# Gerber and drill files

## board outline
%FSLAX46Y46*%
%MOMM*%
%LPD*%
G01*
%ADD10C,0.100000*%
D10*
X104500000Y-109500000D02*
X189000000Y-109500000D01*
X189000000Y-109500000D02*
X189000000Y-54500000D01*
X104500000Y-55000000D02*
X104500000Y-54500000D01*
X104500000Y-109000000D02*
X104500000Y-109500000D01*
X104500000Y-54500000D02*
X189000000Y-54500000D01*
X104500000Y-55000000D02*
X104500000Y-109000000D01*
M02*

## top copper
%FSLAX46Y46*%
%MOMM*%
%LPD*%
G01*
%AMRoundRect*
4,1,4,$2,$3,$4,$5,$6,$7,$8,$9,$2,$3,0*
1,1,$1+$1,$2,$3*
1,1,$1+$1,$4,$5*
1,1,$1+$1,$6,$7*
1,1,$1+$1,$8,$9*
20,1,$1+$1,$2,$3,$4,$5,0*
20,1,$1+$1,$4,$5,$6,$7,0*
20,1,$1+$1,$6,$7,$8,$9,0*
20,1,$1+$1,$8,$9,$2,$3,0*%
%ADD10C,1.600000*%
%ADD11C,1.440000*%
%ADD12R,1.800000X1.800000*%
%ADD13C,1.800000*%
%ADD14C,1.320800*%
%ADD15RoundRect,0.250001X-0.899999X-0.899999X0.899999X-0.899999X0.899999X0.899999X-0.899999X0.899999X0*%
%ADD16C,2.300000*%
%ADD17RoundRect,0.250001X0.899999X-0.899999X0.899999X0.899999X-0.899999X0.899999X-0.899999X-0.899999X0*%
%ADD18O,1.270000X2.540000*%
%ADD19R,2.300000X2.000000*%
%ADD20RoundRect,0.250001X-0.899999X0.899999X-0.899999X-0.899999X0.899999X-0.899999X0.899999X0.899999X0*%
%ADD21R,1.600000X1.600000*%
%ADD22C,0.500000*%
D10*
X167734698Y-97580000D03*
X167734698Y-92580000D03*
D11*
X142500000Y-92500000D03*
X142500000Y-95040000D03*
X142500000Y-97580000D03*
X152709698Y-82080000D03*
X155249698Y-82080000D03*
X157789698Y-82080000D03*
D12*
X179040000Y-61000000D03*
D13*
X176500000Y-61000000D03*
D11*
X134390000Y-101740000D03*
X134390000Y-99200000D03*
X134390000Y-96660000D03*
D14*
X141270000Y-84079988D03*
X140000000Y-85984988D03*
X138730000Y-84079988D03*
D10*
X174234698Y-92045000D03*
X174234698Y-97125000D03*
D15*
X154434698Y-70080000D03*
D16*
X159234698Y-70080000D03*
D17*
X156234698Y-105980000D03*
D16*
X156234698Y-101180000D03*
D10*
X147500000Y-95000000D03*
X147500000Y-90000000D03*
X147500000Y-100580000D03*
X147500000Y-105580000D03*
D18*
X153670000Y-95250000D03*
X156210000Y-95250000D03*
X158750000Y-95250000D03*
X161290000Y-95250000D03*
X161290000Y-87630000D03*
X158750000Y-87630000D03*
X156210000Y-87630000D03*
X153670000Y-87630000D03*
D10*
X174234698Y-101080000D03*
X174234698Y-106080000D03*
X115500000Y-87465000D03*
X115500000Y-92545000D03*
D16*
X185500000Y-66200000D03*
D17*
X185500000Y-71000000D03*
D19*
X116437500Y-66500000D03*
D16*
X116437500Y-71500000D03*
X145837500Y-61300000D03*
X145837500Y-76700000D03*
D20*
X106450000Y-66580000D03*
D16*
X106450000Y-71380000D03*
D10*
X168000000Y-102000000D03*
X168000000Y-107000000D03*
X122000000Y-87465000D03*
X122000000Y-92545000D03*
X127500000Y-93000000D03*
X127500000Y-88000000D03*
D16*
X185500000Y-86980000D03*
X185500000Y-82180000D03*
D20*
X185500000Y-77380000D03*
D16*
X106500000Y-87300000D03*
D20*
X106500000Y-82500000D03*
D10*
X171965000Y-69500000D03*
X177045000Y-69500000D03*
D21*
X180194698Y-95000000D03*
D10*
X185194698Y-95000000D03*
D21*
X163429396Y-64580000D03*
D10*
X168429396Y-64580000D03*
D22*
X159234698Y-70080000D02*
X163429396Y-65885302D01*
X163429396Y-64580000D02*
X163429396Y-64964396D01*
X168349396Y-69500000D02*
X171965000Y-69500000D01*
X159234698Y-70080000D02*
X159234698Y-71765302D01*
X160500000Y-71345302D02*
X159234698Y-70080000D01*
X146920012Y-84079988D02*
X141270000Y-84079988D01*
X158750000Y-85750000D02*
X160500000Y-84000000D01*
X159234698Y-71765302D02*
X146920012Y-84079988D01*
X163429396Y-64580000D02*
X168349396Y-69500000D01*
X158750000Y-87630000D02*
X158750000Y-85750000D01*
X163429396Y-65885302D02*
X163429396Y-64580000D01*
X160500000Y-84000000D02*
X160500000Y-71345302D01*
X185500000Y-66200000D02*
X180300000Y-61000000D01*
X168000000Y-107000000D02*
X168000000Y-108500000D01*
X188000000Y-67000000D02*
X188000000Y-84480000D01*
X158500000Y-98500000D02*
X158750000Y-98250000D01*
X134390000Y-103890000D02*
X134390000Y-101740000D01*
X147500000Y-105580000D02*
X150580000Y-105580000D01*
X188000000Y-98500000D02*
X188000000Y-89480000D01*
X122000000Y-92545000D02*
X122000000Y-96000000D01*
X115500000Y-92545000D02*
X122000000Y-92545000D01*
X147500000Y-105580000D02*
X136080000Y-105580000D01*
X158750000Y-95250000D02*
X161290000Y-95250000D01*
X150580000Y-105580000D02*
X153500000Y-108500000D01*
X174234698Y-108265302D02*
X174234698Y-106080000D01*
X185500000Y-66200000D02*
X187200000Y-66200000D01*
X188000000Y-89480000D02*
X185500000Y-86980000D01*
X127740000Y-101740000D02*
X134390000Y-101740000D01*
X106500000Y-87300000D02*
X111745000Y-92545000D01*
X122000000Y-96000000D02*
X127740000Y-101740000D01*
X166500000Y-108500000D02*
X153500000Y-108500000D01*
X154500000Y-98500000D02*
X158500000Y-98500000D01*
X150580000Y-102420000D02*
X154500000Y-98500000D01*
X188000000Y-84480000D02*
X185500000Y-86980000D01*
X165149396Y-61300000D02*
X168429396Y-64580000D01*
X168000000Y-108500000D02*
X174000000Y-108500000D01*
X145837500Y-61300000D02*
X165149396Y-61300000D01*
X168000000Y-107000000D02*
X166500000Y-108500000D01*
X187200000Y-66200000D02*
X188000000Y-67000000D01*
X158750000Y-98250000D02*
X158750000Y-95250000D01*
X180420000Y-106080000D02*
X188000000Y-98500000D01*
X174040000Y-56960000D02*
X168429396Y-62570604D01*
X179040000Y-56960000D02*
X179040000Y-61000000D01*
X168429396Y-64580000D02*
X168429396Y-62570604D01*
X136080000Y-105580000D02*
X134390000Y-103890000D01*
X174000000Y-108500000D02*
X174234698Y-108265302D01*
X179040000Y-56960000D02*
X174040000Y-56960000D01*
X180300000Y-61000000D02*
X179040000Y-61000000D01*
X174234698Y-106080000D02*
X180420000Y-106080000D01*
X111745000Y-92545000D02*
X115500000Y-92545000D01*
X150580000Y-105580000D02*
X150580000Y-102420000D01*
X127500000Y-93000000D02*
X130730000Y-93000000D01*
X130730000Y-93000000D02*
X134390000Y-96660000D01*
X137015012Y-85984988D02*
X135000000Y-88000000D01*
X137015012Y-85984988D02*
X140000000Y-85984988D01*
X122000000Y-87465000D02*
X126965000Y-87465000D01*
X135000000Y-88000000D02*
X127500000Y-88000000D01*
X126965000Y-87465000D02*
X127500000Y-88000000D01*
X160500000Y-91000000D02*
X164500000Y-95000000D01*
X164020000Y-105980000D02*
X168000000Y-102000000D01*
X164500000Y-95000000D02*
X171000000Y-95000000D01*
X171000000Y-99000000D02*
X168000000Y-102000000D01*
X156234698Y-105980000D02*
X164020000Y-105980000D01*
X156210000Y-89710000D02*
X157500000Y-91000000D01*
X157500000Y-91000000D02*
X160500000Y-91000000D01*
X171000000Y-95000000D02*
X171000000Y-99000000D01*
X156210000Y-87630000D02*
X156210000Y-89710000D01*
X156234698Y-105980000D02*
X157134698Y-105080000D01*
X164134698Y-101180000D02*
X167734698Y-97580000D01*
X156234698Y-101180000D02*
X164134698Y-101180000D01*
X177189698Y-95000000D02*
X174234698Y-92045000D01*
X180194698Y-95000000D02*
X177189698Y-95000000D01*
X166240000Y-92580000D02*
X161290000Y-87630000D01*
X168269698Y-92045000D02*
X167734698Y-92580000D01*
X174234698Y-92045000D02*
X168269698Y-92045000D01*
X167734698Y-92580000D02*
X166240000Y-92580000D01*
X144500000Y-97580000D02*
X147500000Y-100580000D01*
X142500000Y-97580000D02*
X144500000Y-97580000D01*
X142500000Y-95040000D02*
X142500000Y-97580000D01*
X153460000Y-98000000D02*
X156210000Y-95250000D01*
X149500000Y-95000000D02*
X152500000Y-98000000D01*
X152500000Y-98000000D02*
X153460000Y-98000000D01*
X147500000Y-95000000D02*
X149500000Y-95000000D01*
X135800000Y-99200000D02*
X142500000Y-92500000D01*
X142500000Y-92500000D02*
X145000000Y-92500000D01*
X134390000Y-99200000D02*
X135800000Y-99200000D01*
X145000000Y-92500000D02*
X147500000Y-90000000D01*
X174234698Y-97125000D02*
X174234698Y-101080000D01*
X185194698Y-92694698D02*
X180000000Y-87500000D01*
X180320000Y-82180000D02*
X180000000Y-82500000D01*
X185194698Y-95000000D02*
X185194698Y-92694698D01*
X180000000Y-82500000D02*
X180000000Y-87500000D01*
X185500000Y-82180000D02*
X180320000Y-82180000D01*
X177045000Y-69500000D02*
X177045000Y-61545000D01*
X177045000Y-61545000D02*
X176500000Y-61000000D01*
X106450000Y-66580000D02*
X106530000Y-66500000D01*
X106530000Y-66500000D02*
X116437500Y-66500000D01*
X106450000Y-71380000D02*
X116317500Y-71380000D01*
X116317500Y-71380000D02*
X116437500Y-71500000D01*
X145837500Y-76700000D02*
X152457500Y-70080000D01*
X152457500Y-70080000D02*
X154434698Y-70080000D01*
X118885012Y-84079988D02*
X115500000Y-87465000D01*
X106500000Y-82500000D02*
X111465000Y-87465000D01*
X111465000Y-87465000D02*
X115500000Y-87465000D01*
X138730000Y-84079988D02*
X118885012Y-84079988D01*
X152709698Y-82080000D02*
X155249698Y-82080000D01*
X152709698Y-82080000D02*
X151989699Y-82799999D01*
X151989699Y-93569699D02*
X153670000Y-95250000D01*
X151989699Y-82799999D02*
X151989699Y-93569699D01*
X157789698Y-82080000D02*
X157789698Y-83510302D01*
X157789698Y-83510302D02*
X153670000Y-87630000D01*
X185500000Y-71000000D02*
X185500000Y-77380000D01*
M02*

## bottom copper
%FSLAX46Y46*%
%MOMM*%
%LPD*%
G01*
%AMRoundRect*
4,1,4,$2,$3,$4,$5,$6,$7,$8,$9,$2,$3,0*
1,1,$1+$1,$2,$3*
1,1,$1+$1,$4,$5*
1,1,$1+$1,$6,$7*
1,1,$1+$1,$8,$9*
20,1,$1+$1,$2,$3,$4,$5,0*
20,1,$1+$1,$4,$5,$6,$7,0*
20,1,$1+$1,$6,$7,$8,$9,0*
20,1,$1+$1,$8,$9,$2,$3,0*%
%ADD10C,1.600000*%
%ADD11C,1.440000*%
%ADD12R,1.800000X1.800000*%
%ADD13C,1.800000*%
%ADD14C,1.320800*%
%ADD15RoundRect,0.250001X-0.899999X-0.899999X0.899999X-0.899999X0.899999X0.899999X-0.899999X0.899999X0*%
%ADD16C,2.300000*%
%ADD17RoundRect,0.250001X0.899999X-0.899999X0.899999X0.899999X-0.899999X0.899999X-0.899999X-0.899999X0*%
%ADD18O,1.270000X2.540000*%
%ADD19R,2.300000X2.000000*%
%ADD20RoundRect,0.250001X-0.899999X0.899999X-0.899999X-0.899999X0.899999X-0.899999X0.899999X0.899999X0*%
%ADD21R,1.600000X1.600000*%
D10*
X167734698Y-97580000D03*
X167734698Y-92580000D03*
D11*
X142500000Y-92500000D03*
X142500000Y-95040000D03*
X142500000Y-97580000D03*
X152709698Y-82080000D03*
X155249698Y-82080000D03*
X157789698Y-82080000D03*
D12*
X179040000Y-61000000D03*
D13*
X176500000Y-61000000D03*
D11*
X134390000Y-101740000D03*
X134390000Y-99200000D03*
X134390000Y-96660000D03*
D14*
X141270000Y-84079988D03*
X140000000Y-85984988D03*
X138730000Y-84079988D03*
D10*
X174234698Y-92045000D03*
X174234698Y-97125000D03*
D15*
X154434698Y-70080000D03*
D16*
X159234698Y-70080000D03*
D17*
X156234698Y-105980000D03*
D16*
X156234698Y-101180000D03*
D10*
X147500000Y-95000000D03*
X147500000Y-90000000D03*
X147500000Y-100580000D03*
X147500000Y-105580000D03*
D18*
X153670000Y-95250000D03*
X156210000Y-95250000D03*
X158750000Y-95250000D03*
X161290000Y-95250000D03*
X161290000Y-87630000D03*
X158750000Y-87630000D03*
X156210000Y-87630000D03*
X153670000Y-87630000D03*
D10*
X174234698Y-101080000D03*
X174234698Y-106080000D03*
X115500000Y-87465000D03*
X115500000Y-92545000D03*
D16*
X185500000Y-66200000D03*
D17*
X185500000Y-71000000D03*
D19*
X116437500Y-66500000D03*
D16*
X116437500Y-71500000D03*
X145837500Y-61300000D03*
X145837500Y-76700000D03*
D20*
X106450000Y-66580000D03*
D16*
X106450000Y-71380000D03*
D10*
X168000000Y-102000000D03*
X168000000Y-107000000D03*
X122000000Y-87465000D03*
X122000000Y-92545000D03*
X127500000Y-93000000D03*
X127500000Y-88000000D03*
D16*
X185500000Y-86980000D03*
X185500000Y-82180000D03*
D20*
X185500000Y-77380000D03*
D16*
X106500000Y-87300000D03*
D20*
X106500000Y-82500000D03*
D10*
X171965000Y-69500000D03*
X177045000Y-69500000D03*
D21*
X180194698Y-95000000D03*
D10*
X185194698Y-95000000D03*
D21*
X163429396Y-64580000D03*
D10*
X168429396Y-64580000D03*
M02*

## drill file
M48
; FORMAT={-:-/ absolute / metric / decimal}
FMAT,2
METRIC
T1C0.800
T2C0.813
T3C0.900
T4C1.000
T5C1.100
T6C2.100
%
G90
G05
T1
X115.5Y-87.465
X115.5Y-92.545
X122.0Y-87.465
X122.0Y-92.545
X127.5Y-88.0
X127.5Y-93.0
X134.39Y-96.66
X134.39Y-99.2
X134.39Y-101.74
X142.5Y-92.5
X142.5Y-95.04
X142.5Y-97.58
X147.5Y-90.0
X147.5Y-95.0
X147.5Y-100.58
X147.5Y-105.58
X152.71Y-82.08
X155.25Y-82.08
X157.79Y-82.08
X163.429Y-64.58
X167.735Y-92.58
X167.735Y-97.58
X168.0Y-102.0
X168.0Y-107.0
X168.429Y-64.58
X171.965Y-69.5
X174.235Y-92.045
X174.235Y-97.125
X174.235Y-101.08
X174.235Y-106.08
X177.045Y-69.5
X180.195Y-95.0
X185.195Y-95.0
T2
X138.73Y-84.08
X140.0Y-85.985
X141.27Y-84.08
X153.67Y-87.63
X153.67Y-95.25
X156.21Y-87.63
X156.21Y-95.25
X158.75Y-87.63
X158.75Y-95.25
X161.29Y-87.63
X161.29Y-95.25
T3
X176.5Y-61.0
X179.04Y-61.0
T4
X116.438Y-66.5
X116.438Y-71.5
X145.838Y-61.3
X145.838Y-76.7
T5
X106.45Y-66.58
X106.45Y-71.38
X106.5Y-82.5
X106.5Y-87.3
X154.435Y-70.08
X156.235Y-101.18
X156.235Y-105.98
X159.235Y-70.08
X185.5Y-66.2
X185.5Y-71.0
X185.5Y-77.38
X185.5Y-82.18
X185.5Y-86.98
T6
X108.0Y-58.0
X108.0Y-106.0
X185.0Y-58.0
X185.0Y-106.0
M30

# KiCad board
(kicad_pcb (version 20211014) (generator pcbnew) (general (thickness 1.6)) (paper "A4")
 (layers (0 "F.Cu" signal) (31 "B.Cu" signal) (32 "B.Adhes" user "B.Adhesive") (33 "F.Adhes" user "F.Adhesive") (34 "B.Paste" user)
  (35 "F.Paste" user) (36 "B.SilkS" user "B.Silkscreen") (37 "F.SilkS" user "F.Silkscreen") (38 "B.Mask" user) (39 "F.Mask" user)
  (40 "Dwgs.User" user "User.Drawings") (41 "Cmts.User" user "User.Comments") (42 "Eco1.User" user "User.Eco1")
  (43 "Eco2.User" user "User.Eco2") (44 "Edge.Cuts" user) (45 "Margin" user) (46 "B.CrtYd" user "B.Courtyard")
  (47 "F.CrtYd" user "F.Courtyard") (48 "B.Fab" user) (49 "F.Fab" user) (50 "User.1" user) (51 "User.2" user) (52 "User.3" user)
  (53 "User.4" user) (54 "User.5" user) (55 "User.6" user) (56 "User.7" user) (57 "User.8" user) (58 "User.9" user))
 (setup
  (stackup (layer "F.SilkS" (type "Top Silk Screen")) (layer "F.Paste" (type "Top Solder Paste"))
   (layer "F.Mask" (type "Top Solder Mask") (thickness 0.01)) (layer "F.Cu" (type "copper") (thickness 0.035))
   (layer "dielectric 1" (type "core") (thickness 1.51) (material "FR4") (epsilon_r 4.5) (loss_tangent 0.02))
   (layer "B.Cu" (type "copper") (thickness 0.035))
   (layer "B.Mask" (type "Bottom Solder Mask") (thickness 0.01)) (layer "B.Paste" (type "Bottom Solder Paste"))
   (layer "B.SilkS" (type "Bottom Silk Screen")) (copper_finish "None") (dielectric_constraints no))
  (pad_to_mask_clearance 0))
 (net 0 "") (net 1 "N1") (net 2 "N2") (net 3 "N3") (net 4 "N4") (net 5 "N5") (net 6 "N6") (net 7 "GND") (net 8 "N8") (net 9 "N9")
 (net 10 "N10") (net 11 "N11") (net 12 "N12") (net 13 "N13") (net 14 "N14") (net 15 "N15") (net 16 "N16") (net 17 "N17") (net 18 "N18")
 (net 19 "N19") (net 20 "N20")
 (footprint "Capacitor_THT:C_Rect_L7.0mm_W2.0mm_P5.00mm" (layer "F.Cu") (at 167.734698 97.58 90)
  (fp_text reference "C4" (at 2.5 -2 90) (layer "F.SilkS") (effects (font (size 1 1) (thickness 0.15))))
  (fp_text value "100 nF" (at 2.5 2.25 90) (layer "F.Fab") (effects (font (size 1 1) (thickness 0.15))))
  (pad "1" thru_hole circle (at 0 0 90) (size 1.6 1.6) (drill 0.8) (layers *.Cu *.Mask) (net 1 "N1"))
  (pad "2" thru_hole circle (at 5 0 90) (size 1.6 1.6) (drill 0.8) (layers *.Cu *.Mask) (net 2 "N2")))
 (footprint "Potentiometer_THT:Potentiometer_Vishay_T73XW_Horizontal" (layer "F.Cu") (at 142.5 92.5)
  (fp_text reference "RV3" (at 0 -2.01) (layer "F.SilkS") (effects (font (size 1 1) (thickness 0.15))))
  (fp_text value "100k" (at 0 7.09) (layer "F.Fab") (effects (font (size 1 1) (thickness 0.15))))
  (pad "1" thru_hole circle (at 0 0) (size 1.44 1.44) (drill 0.8) (layers *.Cu *.Mask) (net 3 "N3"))
  (pad "2" thru_hole circle (at 0 2.54) (size 1.44 1.44) (drill 0.8) (layers *.Cu *.Mask) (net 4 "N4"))
  (pad "3" thru_hole circle (at 0 5.08) (size 1.44 1.44) (drill 0.8) (layers *.Cu *.Mask) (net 4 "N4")))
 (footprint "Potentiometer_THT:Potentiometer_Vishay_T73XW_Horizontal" (layer "F.Cu") (at 152.709698 82.08 90)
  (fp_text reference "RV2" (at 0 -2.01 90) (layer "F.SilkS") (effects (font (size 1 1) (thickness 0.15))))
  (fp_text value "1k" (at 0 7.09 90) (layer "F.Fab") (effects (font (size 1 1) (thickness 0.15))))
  (pad "1" thru_hole circle (at 0 0 90) (size 1.44 1.44) (drill 0.8) (layers *.Cu *.Mask) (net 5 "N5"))
  (pad "2" thru_hole circle (at 0 2.54 90) (size 1.44 1.44) (drill 0.8) (layers *.Cu *.Mask) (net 5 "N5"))
  (pad "3" thru_hole circle (at 0 5.08 90) (size 1.44 1.44) (drill 0.8) (layers *.Cu *.Mask) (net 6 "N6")))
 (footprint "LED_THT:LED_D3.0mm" (layer "F.Cu") (at 179.04 61 180)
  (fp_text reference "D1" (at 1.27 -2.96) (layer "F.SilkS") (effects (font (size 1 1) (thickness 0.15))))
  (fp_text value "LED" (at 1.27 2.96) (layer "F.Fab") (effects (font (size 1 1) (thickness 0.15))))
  (pad "1" thru_hole rect (at 0 0 180) (size 1.8 1.8) (drill 0.9) (layers *.Cu *.Mask) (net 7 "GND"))
  (pad "2" thru_hole circle (at 2.54 0 180) (size 1.8 1.8) (drill 0.9) (layers *.Cu *.Mask) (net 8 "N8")))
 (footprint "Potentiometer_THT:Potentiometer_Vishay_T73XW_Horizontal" (layer "F.Cu") (at 134.39 101.74 180)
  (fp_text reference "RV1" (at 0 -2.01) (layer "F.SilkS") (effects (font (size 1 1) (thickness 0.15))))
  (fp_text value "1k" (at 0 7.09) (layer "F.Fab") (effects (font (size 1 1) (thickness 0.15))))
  (pad "1" thru_hole circle (at 0 0 180) (size 1.44 1.44) (drill 0.8) (layers *.Cu *.Mask) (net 7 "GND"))
  (pad "2" thru_hole circle (at 0 2.54 180) (size 1.44 1.44) (drill 0.8) (layers *.Cu *.Mask) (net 3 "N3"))
  (pad "3" thru_hole circle (at 0 5.08 180) (size 1.44 1.44) (drill 0.8) (layers *.Cu *.Mask) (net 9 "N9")))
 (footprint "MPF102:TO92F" (layer "F.Cu") (at 140 84.079988 180)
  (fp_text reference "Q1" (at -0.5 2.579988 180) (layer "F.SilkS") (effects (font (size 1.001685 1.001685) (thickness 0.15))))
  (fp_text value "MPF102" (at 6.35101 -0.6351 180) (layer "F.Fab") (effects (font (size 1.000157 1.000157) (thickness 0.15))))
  (pad "1" thru_hole circle locked (at -1.27 0 180) (size 1.3208 1.3208) (drill 0.8128) (layers *.Cu *.Mask) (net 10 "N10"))
  (pad "2" thru_hole circle locked (at 0 -1.905 180) (size 1.3208 1.3208) (drill 0.8128) (layers *.Cu *.Mask) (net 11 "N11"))
  (pad "3" thru_hole circle locked (at 1.27 0 180) (size 1.3208 1.3208) (drill 0.8128) (layers *.Cu *.Mask) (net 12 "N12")))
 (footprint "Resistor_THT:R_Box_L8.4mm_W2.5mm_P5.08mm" (layer "F.Cu") (at 174.234698 92.045 -90)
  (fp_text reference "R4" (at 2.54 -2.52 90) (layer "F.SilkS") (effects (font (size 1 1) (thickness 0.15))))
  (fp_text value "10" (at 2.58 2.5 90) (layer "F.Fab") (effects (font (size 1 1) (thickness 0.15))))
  (pad "1" thru_hole circle (at 0 0 270) (size 1.6 1.6) (drill 0.8) (layers *.Cu *.Mask) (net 2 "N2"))
  (pad "2" thru_hole circle (at 5.08 0 270) (size 1.6 1.6) (drill 0.8) (layers *.Cu *.Mask) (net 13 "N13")))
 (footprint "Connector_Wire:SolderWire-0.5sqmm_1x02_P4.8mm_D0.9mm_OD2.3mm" (layer "F.Cu") (at 154.434698 70.08)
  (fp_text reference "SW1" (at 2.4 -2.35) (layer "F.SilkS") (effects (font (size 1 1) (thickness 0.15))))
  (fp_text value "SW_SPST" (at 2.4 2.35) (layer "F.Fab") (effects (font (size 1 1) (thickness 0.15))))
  (pad "1" thru_hole roundrect (at 0 0) (size 2.3 2.3) (drill 1.1) (layers *.Cu *.Mask) (roundrect_rratio 0.108696) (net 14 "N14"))
  (pad "2" thru_hole circle (at 4.8 0) (size 2.3 2.3) (drill 1.1) (layers *.Cu *.Mask) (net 10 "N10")))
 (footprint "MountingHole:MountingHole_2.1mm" (layer "F.Cu") (at 185 106)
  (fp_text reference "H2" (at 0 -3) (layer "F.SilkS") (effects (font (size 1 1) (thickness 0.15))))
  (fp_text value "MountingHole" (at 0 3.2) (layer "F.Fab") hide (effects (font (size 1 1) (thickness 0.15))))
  (pad "" np_thru_hole circle (at 0 0) (size 2.1 2.1) (drill 2.1) (layers *.Cu *.Mask)))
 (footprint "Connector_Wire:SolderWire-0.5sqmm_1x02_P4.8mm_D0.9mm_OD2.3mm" (layer "F.Cu") (at 156.234698 105.98 90)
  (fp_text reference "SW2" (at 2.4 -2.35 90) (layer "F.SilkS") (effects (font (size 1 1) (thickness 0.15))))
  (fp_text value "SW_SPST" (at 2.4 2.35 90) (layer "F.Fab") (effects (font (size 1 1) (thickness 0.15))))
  (pad "1" thru_hole roundrect (at 0 0 90) (size 2.3 2.3) (drill 1.1) (layers *.Cu *.Mask) (roundrect_rratio 0.108696) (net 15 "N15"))
  (pad "2" thru_hole circle (at 4.8 0 90) (size 2.3 2.3) (drill 1.1) (layers *.Cu *.Mask) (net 1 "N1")))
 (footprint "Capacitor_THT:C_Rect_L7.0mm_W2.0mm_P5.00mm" (layer "F.Cu") (at 147.5 95 90)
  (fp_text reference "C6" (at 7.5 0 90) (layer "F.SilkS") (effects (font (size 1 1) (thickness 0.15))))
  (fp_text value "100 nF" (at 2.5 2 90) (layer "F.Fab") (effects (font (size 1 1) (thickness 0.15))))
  (pad "1" thru_hole circle (at 0 0 90) (size 1.6 1.6) (drill 0.8) (layers *.Cu *.Mask) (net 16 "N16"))
  (pad "2" thru_hole circle (at 5 0 90) (size 1.6 1.6) (drill 0.8) (layers *.Cu *.Mask) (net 3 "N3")))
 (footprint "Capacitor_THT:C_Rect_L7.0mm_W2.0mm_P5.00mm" (layer "F.Cu") (at 147.5 100.58 -90)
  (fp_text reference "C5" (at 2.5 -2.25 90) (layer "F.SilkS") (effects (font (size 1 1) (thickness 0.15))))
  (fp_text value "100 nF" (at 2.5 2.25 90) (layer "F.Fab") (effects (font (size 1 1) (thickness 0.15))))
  (pad "1" thru_hole circle (at 0 0 270) (size 1.6 1.6) (drill 0.8) (layers *.Cu *.Mask) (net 4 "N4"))
  (pad "2" thru_hole circle (at 5 0 270) (size 1.6 1.6) (drill 0.8) (layers *.Cu *.Mask) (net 7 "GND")))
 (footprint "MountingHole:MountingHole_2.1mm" (layer "F.Cu") (at 108 106)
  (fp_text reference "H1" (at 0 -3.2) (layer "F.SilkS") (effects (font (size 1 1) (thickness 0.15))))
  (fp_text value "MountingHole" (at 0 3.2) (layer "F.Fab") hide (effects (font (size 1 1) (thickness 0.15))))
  (pad "" np_thru_hole circle (at 0 0) (size 2.1 2.1) (drill 2.1) (layers *.Cu *.Mask)))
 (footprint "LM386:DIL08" (layer "F.Cu") (at 157.48 91.44)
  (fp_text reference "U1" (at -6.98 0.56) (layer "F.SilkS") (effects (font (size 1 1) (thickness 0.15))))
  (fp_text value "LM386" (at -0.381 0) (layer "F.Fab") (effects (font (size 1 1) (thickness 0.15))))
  (pad "1" thru_hole oval locked (at -3.81 3.81) (size 1.27 2.54) (drill 0.8128) (layers *.Cu *.Mask) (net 5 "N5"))
  (pad "2" thru_hole oval locked (at -1.27 3.81) (size 1.27 2.54) (drill 0.8128) (layers *.Cu *.Mask) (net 16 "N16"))
  (pad "3" thru_hole oval locked (at 1.27 3.81) (size 1.27 2.54) (drill 0.8128) (layers *.Cu *.Mask) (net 7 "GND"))
  (pad "4" thru_hole oval locked (at 3.81 3.81) (size 1.27 2.54) (drill 0.8128) (layers *.Cu *.Mask) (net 7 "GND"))
  (pad "5" thru_hole oval locked (at 3.81 -3.81) (size 1.27 2.54) (drill 0.8128) (layers *.Cu *.Mask) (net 2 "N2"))
  (pad "6" thru_hole oval locked (at 1.27 -3.81) (size 1.27 2.54) (drill 0.8128) (layers *.Cu *.Mask) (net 10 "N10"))
  (pad "7" thru_hole oval locked (at -1.27 -3.81) (size 1.27 2.54) (drill 0.8128) (layers *.Cu *.Mask) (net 15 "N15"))
  (pad "8" thru_hole oval locked (at -3.81 -3.81) (size 1.27 2.54) (drill 0.8128) (layers *.Cu *.Mask) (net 6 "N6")))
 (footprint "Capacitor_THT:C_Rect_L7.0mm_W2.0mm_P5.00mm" (layer "F.Cu") (at 174.234698 101.08 -90)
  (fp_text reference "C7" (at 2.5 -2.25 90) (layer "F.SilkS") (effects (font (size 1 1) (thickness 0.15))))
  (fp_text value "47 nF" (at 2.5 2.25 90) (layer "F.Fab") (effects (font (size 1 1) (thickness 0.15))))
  (pad "1" thru_hole circle (at 0 0 270) (size 1.6 1.6) (drill 0.8) (layers *.Cu *.Mask) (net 13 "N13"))
  (pad "2" thru_hole circle (at 5 0 270) (size 1.6 1.6) (drill 0.8) (layers *.Cu *.Mask) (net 7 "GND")))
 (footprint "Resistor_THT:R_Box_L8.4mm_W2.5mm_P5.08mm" (layer "F.Cu") (at 115.5 87.465 -90)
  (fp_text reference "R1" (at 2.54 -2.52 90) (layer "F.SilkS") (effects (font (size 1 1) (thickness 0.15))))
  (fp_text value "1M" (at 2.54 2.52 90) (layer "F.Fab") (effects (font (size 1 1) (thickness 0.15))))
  (pad "1" thru_hole circle (at 0 0 270) (size 1.6 1.6) (drill 0.8) (layers *.Cu *.Mask) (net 12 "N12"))
  (pad "2" thru_hole circle (at 5.08 0 270) (size 1.6 1.6) (drill 0.8) (layers *.Cu *.Mask) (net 7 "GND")))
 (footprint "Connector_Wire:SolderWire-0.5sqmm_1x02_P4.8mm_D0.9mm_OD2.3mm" (layer "F.Cu") (at 185.5 71 90)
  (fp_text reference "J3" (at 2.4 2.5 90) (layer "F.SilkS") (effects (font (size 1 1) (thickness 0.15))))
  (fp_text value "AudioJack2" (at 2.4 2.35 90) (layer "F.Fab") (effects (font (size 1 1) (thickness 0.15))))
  (pad "S" thru_hole circle (at 4.8 0 90) (size 2.3 2.3) (drill 1.1) (layers *.Cu *.Mask) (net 7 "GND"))
  (pad "T" thru_hole roundrect (at 0 0 90) (size 2.3 2.3) (drill 1.1) (layers *.Cu *.Mask) (roundrect_rratio 0.108696) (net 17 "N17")))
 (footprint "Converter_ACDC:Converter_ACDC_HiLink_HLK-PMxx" (layer "F.Cu") (at 116.4375 66.5)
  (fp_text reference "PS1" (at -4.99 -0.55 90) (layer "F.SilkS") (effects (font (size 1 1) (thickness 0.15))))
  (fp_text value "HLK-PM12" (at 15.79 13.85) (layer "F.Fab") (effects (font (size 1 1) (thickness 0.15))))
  (pad "1" thru_hole rect (at 0 0) (size 2.3 2) (drill 1) (layers *.Cu *.Mask) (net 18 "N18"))
  (pad "2" thru_hole circle (at 0 5) (size 2.3 2.3) (drill 1) (layers *.Cu *.Mask) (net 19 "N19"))
  (pad "3" thru_hole circle (at 29.4 -5.2) (size 2.3 2.3) (drill 1) (layers *.Cu *.Mask) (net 7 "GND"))
  (pad "4" thru_hole circle (at 29.4 10.2) (size 2.3 2.3) (drill 1) (layers *.Cu *.Mask) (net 14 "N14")))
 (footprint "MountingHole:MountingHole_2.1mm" (layer "F.Cu") (at 108 58)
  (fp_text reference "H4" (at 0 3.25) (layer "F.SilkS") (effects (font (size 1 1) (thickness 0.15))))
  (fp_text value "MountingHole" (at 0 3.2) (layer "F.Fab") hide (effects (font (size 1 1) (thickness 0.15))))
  (pad "" np_thru_hole circle (at 0 0) (size 2.1 2.1) (drill 2.1) (layers *.Cu *.Mask)))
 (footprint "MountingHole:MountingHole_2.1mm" (layer "F.Cu") (at 185 58)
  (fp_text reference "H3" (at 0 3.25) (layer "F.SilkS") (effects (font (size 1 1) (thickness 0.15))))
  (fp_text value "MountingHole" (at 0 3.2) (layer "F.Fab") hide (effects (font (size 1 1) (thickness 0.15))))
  (pad "" np_thru_hole circle (at 0 0) (size 2.1 2.1) (drill 2.1) (layers *.Cu *.Mask)))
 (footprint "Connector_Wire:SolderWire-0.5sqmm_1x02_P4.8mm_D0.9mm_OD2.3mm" (layer "F.Cu") (at 106.45 66.58 -90)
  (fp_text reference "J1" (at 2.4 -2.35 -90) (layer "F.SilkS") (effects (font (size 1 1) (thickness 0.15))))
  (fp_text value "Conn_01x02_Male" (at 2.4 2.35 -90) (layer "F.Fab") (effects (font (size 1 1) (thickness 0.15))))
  (pad "1" thru_hole roundrect (at 0 0 270) (size 2.3 2.3) (drill 1.1) (layers *.Cu *.Mask) (roundrect_rratio 0.108696) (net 18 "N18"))
  (pad "2" thru_hole circle (at 4.8 0 270) (size 2.3 2.3) (drill 1.1) (layers *.Cu *.Mask) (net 19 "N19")))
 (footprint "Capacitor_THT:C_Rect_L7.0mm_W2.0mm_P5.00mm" (layer "F.Cu") (at 168 102 -90)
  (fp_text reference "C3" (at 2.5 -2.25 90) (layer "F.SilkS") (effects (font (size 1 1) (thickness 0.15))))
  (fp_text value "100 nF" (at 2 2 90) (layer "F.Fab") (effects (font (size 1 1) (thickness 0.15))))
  (pad "1" thru_hole circle (at 0 0 270) (size 1.6 1.6) (drill 0.8) (layers *.Cu *.Mask) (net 15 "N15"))
  (pad "2" thru_hole circle (at 5 0 270) (size 1.6 1.6) (drill 0.8) (layers *.Cu *.Mask) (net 7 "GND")))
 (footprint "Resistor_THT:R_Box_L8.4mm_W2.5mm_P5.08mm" (layer "F.Cu") (at 122 87.465 -90)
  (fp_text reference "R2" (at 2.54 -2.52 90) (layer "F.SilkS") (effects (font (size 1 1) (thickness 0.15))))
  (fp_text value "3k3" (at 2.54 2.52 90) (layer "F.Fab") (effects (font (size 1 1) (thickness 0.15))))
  (pad "1" thru_hole circle (at 0 0 270) (size 1.6 1.6) (drill 0.8) (layers *.Cu *.Mask) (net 11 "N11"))
  (pad "2" thru_hole circle (at 5.08 0 270) (size 1.6 1.6) (drill 0.8) (layers *.Cu *.Mask) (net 7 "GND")))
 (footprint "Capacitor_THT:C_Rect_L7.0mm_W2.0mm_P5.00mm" (layer "F.Cu") (at 127.5 93 90)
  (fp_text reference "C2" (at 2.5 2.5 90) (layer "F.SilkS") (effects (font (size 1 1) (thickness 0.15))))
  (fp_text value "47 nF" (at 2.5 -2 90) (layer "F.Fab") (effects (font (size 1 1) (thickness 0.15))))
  (pad "1" thru_hole circle (at 0 0 90) (size 1.6 1.6) (drill 0.8) (layers *.Cu *.Mask) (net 9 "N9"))
  (pad "2" thru_hole circle (at 5 0 90) (size 1.6 1.6) (drill 0.8) (layers *.Cu *.Mask) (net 11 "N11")))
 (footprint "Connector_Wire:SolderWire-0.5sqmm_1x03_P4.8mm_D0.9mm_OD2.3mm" (layer "F.Cu") (at 185.5 77.38 -90)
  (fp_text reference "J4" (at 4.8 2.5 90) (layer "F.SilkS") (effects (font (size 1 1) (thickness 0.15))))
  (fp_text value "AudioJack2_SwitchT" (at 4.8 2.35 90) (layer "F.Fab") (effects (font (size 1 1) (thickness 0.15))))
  (pad "S" thru_hole circle (at 9.6 0 270) (size 2.3 2.3) (drill 1.1) (layers *.Cu *.Mask) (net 7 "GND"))
  (pad "T" thru_hole circle (at 4.8 0 270) (size 2.3 2.3) (drill 1.1) (layers *.Cu *.Mask) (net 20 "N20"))
  (pad "TN" thru_hole roundrect (at 0 0 270) (size 2.3 2.3) (drill 1.1) (layers *.Cu *.Mask) (roundrect_rratio 0.108696) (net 17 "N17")))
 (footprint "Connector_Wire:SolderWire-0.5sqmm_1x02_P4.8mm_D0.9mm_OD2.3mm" (layer "F.Cu") (at 106.5 82.5 -90)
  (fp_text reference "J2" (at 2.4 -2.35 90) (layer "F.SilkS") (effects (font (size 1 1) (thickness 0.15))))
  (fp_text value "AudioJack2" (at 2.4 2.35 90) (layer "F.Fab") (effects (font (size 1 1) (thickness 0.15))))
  (pad "S" thru_hole circle (at 4.8 0 270) (size 2.3 2.3) (drill 1.1) (layers *.Cu *.Mask) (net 7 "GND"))
  (pad "T" thru_hole roundrect (at 0 0 270) (size 2.3 2.3) (drill 1.1) (layers *.Cu *.Mask) (roundrect_rratio 0.108696) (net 12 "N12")))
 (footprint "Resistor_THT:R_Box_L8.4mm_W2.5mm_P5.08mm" (layer "F.Cu") (at 171.965 69.5)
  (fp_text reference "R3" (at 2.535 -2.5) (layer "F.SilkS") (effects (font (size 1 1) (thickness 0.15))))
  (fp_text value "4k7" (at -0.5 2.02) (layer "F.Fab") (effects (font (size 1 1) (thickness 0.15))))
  (pad "1" thru_hole circle (at 0 0) (size 1.6 1.6) (drill 0.8) (layers *.Cu *.Mask) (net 10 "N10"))
  (pad "2" thru_hole circle (at 5.08 0) (size 1.6 1.6) (drill 0.8) (layers *.Cu *.Mask) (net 8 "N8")))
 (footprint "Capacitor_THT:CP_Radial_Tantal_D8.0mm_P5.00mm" (layer "F.Cu") (at 180.194698 95)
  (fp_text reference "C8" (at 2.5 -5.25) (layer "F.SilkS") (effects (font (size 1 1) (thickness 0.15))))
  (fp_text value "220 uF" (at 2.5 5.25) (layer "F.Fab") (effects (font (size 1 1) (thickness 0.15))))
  (pad "1" thru_hole rect (at 0 0) (size 1.6 1.6) (drill 0.8) (layers *.Cu *.Mask) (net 2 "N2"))
  (pad "2" thru_hole circle (at 5 0) (size 1.6 1.6) (drill 0.8) (layers *.Cu *.Mask) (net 20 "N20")))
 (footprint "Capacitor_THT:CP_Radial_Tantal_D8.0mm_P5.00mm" (layer "F.Cu") (at 163.429396 64.58)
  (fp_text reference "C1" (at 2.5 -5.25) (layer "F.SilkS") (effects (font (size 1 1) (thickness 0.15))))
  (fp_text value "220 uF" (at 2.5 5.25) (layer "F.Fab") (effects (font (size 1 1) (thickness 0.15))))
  (pad "1" thru_hole rect (at 0 0) (size 1.6 1.6) (drill 0.8) (layers *.Cu *.Mask) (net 10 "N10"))
  (pad "2" thru_hole circle (at 5 0) (size 1.6 1.6) (drill 0.8) (layers *.Cu *.Mask) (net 7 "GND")))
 (gr_line (start 104.5 109.5) (end 189 109.5) (layer "Edge.Cuts") (width 0.1))
 (gr_line (start 189 109.5) (end 189 54.5) (layer "Edge.Cuts") (width 0.1))
 (gr_line (start 104.5 55) (end 104.5 54.5) (layer "Edge.Cuts") (width 0.1))
 (gr_line (start 104.5 109) (end 104.5 109.5) (layer "Edge.Cuts") (width 0.1))
 (gr_line (start 104.5 54.5) (end 189 54.5) (layer "Edge.Cuts") (width 0.1))
 (gr_line (start 104.5 55) (end 104.5 109) (layer "Edge.Cuts") (width 0.1))
 (segment (start 159.234698 70.08) (end 163.429396 65.885302) (width 0.5) (layer "F.Cu") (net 10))
 (segment (start 163.429396 64.58) (end 163.429396 64.964396) (width 0.5) (layer "F.Cu") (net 10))
 (segment (start 168.349396 69.5) (end 171.965 69.5) (width 0.5) (layer "F.Cu") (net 10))
 (segment (start 159.234698 70.08) (end 159.234698 71.765302) (width 0.5) (layer "F.Cu") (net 10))
 (segment (start 160.5 71.345302) (end 159.234698 70.08) (width 0.5) (layer "F.Cu") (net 10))
 (segment (start 146.920012 84.079988) (end 141.27 84.079988) (width 0.5) (layer "F.Cu") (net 10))
 (segment (start 158.75 85.75) (end 160.5 84) (width 0.5) (layer "F.Cu") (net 10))
 (segment (start 159.234698 71.765302) (end 146.920012 84.079988) (width 0.5) (layer "F.Cu") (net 10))
 (segment (start 163.429396 64.58) (end 168.349396 69.5) (width 0.5) (layer "F.Cu") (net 10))
 (segment (start 158.75 87.63) (end 158.75 85.75) (width 0.5) (layer "F.Cu") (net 10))
 (segment (start 163.429396 65.885302) (end 163.429396 64.58) (width 0.5) (layer "F.Cu") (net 10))
 (segment (start 160.5 84) (end 160.5 71.345302) (width 0.5) (layer "F.Cu") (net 10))
 (segment (start 185.5 66.2) (end 180.3 61) (width 0.5) (layer "F.Cu") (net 7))
 (segment (start 168 107) (end 168 108.5) (width 0.5) (layer "F.Cu") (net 7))
 (segment (start 188 67) (end 188 84.48) (width 0.5) (layer "F.Cu") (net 7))
 (segment (start 158.5 98.5) (end 158.75 98.25) (width 0.5) (layer "F.Cu") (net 7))
 (segment (start 134.39 103.89) (end 134.39 101.74) (width 0.5) (layer "F.Cu") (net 7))
 (segment (start 147.5 105.58) (end 150.58 105.58) (width 0.5) (layer "F.Cu") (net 7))
 (segment (start 188 98.5) (end 188 89.48) (width 0.5) (layer "F.Cu") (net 7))
 (segment (start 122 92.545) (end 122 96) (width 0.5) (layer "F.Cu") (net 7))
 (segment (start 115.5 92.545) (end 122 92.545) (width 0.5) (layer "F.Cu") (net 7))
 (segment (start 147.5 105.58) (end 136.08 105.58) (width 0.5) (layer "F.Cu") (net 7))
 (segment (start 158.75 95.25) (end 161.29 95.25) (width 0.5) (layer "F.Cu") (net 7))
 (segment (start 150.58 105.58) (end 153.5 108.5) (width 0.5) (layer "F.Cu") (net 7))
 (segment (start 174.234698 108.265302) (end 174.234698 106.08) (width 0.5) (layer "F.Cu") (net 7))
 (segment (start 185.5 66.2) (end 187.2 66.2) (width 0.5) (layer "F.Cu") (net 7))
 (segment (start 188 89.48) (end 185.5 86.98) (width 0.5) (layer "F.Cu") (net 7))
 (segment (start 127.74 101.74) (end 134.39 101.74) (width 0.5) (layer "F.Cu") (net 7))
 (segment (start 106.5 87.3) (end 111.745 92.545) (width 0.5) (layer "F.Cu") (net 7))
 (segment (start 122 96) (end 127.74 101.74) (width 0.5) (layer "F.Cu") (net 7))
 (segment (start 166.5 108.5) (end 153.5 108.5) (width 0.5) (layer "F.Cu") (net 7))
 (segment (start 154.5 98.5) (end 158.5 98.5) (width 0.5) (layer "F.Cu") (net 7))
 (segment (start 150.58 102.42) (end 154.5 98.5) (width 0.5) (layer "F.Cu") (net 7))
 (segment (start 188 84.48) (end 185.5 86.98) (width 0.5) (layer "F.Cu") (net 7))
 (segment (start 165.149396 61.3) (end 168.429396 64.58) (width 0.5) (layer "F.Cu") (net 7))
 (segment (start 168 108.5) (end 174 108.5) (width 0.5) (layer "F.Cu") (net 7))
 (segment (start 145.8375 61.3) (end 165.149396 61.3) (width 0.5) (layer "F.Cu") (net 7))
 (segment (start 168 107) (end 166.5 108.5) (width 0.5) (layer "F.Cu") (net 7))
 (segment (start 187.2 66.2) (end 188 67) (width 0.5) (layer "F.Cu") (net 7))
 (segment (start 158.75 98.25) (end 158.75 95.25) (width 0.5) (layer "F.Cu") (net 7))
 (segment (start 180.42 106.08) (end 188 98.5) (width 0.5) (layer "F.Cu") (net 7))
 (segment (start 174.04 56.96) (end 168.429396 62.570604) (width 0.5) (layer "F.Cu") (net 7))
 (segment (start 179.04 56.96) (end 179.04 61) (width 0.5) (layer "F.Cu") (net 7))
 (segment (start 168.429396 64.58) (end 168.429396 62.570604) (width 0.5) (layer "F.Cu") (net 7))
 (segment (start 136.08 105.58) (end 134.39 103.89) (width 0.5) (layer "F.Cu") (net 7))
 (segment (start 174 108.5) (end 174.234698 108.265302) (width 0.5) (layer "F.Cu") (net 7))
 (segment (start 179.04 56.96) (end 174.04 56.96) (width 0.5) (layer "F.Cu") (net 7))
 (segment (start 180.3 61) (end 179.04 61) (width 0.5) (layer "F.Cu") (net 7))
 (segment (start 174.234698 106.08) (end 180.42 106.08) (width 0.5) (layer "F.Cu") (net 7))
 (segment (start 111.745 92.545) (end 115.5 92.545) (width 0.5) (layer "F.Cu") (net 7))
 (segment (start 150.58 105.58) (end 150.58 102.42) (width 0.5) (layer "F.Cu") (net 7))
 (segment (start 127.5 93) (end 130.73 93) (width 0.5) (layer "F.Cu") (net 9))
 (segment (start 130.73 93) (end 134.39 96.66) (width 0.5) (layer "F.Cu") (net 9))
 (segment (start 137.015012 85.984988) (end 135 88) (width 0.5) (layer "F.Cu") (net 11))
 (segment (start 137.015012 85.984988) (end 140 85.984988) (width 0.5) (layer "F.Cu") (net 11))
 (segment (start 122 87.465) (end 126.965 87.465) (width 0.5) (layer "F.Cu") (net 11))
 (segment (start 135 88) (end 127.5 88) (width 0.5) (layer "F.Cu") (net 11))
 (segment (start 126.965 87.465) (end 127.5 88) (width 0.5) (layer "F.Cu") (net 11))
 (segment (start 160.5 91) (end 164.5 95) (width 0.5) (layer "F.Cu") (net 15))
 (segment (start 164.02 105.98) (end 168 102) (width 0.5) (layer "F.Cu") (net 15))
 (segment (start 164.5 95) (end 171 95) (width 0.5) (layer "F.Cu") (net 15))
 (segment (start 171 99) (end 168 102) (width 0.5) (layer "F.Cu") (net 15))
 (segment (start 156.234698 105.98) (end 164.02 105.98) (width 0.5) (layer "F.Cu") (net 15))
 (segment (start 156.21 89.71) (end 157.5 91) (width 0.5) (layer "F.Cu") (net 15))
 (segment (start 157.5 91) (end 160.5 91) (width 0.5) (layer "F.Cu") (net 15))
 (segment (start 171 95) (end 171 99) (width 0.5) (layer "F.Cu") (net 15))
 (segment (start 156.21 87.63) (end 156.21 89.71) (width 0.5) (layer "F.Cu") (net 15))
 (segment (start 156.234698 105.98) (end 157.134698 105.08) (width 0.5) (layer "F.Cu") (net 15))
 (segment (start 164.134698 101.18) (end 167.734698 97.58) (width 0.5) (layer "F.Cu") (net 1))
 (segment (start 156.234698 101.18) (end 164.134698 101.18) (width 0.5) (layer "F.Cu") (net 1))
 (segment (start 177.189698 95) (end 174.234698 92.045) (width 0.5) (layer "F.Cu") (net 2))
 (segment (start 180.194698 95) (end 177.189698 95) (width 0.5) (layer "F.Cu") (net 2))
 (segment (start 166.24 92.58) (end 161.29 87.63) (width 0.5) (layer "F.Cu") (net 2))
 (segment (start 168.269698 92.045) (end 167.734698 92.58) (width 0.5) (layer "F.Cu") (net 2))
 (segment (start 174.234698 92.045) (end 168.269698 92.045) (width 0.5) (layer "F.Cu") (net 2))
 (segment (start 167.734698 92.58) (end 166.24 92.58) (width 0.5) (layer "F.Cu") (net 2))
 (segment (start 144.5 97.58) (end 147.5 100.58) (width 0.5) (layer "F.Cu") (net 4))
 (segment (start 142.5 97.58) (end 144.5 97.58) (width 0.5) (layer "F.Cu") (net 4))
 (segment (start 142.5 95.04) (end 142.5 97.58) (width 0.5) (layer "F.Cu") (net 4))
 (segment (start 153.46 98) (end 156.21 95.25) (width 0.5) (layer "F.Cu") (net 16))
 (segment (start 149.5 95) (end 152.5 98) (width 0.5) (layer "F.Cu") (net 16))
 (segment (start 152.5 98) (end 153.46 98) (width 0.5) (layer "F.Cu") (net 16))
 (segment (start 147.5 95) (end 149.5 95) (width 0.5) (layer "F.Cu") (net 16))
 (segment (start 135.8 99.2) (end 142.5 92.5) (width 0.5) (layer "F.Cu") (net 3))
 (segment (start 142.5 92.5) (end 145 92.5) (width 0.5) (layer "F.Cu") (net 3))
 (segment (start 134.39 99.2) (end 135.8 99.2) (width 0.5) (layer "F.Cu") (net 3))
 (segment (start 145 92.5) (end 147.5 90) (width 0.5) (layer "F.Cu") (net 3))
 (segment (start 174.234698 97.125) (end 174.234698 101.08) (width 0.5) (layer "F.Cu") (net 13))
 (segment (start 185.194698 92.694698) (end 180 87.5) (width 0.5) (layer "F.Cu") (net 20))
 (segment (start 180.32 82.18) (end 180 82.5) (width 0.5) (layer "F.Cu") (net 20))
 (segment (start 185.194698 95) (end 185.194698 92.694698) (width 0.5) (layer "F.Cu") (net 20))
 (segment (start 180 82.5) (end 180 87.5) (width 0.5) (layer "F.Cu") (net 20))
 (segment (start 185.5 82.18) (end 180.32 82.18) (width 0.5) (layer "F.Cu") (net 20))
 (segment (start 177.045 69.5) (end 177.045 61.545) (width 0.5) (layer "F.Cu") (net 8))
 (segment (start 177.045 61.545) (end 176.5 61) (width 0.5) (layer "F.Cu") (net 8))
 (segment (start 106.45 66.58) (end 106.53 66.5) (width 0.5) (layer "F.Cu") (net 18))
 (segment (start 106.53 66.5) (end 116.4375 66.5) (width 0.5) (layer "F.Cu") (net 18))
 (segment (start 106.45 71.38) (end 116.3175 71.38) (width 0.5) (layer "F.Cu") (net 19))
 (segment (start 116.3175 71.38) (end 116.4375 71.5) (width 0.5) (layer "F.Cu") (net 19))
 (segment (start 145.8375 76.7) (end 152.4575 70.08) (width 0.5) (layer "F.Cu") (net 14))
 (segment (start 152.4575 70.08) (end 154.434698 70.08) (width 0.5) (layer "F.Cu") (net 14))
 (segment (start 118.885012 84.079988) (end 115.5 87.465) (width 0.5) (layer "F.Cu") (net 12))
 (segment (start 106.5 82.5) (end 111.465 87.465) (width 0.5) (layer "F.Cu") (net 12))
 (segment (start 111.465 87.465) (end 115.5 87.465) (width 0.5) (layer "F.Cu") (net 12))
 (segment (start 138.73 84.079988) (end 118.885012 84.079988) (width 0.5) (layer "F.Cu") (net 12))
 (segment (start 152.709698 82.08) (end 155.249698 82.08) (width 0.5) (layer "F.Cu") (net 5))
 (segment (start 152.709698 82.08) (end 151.989699 82.799999) (width 0.5) (layer "F.Cu") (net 5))
 (segment (start 151.989699 93.569699) (end 153.67 95.25) (width 0.5) (layer "F.Cu") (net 5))
 (segment (start 151.989699 82.799999) (end 151.989699 93.569699) (width 0.5) (layer "F.Cu") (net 5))
 (segment (start 157.789698 82.08) (end 157.789698 83.510302) (width 0.5) (layer "F.Cu") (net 6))
 (segment (start 157.789698 83.510302) (end 153.67 87.63) (width 0.5) (layer "F.Cu") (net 6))
 (segment (start 185.5 71) (end 185.5 77.38) (width 0.5) (layer "F.Cu") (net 17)))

